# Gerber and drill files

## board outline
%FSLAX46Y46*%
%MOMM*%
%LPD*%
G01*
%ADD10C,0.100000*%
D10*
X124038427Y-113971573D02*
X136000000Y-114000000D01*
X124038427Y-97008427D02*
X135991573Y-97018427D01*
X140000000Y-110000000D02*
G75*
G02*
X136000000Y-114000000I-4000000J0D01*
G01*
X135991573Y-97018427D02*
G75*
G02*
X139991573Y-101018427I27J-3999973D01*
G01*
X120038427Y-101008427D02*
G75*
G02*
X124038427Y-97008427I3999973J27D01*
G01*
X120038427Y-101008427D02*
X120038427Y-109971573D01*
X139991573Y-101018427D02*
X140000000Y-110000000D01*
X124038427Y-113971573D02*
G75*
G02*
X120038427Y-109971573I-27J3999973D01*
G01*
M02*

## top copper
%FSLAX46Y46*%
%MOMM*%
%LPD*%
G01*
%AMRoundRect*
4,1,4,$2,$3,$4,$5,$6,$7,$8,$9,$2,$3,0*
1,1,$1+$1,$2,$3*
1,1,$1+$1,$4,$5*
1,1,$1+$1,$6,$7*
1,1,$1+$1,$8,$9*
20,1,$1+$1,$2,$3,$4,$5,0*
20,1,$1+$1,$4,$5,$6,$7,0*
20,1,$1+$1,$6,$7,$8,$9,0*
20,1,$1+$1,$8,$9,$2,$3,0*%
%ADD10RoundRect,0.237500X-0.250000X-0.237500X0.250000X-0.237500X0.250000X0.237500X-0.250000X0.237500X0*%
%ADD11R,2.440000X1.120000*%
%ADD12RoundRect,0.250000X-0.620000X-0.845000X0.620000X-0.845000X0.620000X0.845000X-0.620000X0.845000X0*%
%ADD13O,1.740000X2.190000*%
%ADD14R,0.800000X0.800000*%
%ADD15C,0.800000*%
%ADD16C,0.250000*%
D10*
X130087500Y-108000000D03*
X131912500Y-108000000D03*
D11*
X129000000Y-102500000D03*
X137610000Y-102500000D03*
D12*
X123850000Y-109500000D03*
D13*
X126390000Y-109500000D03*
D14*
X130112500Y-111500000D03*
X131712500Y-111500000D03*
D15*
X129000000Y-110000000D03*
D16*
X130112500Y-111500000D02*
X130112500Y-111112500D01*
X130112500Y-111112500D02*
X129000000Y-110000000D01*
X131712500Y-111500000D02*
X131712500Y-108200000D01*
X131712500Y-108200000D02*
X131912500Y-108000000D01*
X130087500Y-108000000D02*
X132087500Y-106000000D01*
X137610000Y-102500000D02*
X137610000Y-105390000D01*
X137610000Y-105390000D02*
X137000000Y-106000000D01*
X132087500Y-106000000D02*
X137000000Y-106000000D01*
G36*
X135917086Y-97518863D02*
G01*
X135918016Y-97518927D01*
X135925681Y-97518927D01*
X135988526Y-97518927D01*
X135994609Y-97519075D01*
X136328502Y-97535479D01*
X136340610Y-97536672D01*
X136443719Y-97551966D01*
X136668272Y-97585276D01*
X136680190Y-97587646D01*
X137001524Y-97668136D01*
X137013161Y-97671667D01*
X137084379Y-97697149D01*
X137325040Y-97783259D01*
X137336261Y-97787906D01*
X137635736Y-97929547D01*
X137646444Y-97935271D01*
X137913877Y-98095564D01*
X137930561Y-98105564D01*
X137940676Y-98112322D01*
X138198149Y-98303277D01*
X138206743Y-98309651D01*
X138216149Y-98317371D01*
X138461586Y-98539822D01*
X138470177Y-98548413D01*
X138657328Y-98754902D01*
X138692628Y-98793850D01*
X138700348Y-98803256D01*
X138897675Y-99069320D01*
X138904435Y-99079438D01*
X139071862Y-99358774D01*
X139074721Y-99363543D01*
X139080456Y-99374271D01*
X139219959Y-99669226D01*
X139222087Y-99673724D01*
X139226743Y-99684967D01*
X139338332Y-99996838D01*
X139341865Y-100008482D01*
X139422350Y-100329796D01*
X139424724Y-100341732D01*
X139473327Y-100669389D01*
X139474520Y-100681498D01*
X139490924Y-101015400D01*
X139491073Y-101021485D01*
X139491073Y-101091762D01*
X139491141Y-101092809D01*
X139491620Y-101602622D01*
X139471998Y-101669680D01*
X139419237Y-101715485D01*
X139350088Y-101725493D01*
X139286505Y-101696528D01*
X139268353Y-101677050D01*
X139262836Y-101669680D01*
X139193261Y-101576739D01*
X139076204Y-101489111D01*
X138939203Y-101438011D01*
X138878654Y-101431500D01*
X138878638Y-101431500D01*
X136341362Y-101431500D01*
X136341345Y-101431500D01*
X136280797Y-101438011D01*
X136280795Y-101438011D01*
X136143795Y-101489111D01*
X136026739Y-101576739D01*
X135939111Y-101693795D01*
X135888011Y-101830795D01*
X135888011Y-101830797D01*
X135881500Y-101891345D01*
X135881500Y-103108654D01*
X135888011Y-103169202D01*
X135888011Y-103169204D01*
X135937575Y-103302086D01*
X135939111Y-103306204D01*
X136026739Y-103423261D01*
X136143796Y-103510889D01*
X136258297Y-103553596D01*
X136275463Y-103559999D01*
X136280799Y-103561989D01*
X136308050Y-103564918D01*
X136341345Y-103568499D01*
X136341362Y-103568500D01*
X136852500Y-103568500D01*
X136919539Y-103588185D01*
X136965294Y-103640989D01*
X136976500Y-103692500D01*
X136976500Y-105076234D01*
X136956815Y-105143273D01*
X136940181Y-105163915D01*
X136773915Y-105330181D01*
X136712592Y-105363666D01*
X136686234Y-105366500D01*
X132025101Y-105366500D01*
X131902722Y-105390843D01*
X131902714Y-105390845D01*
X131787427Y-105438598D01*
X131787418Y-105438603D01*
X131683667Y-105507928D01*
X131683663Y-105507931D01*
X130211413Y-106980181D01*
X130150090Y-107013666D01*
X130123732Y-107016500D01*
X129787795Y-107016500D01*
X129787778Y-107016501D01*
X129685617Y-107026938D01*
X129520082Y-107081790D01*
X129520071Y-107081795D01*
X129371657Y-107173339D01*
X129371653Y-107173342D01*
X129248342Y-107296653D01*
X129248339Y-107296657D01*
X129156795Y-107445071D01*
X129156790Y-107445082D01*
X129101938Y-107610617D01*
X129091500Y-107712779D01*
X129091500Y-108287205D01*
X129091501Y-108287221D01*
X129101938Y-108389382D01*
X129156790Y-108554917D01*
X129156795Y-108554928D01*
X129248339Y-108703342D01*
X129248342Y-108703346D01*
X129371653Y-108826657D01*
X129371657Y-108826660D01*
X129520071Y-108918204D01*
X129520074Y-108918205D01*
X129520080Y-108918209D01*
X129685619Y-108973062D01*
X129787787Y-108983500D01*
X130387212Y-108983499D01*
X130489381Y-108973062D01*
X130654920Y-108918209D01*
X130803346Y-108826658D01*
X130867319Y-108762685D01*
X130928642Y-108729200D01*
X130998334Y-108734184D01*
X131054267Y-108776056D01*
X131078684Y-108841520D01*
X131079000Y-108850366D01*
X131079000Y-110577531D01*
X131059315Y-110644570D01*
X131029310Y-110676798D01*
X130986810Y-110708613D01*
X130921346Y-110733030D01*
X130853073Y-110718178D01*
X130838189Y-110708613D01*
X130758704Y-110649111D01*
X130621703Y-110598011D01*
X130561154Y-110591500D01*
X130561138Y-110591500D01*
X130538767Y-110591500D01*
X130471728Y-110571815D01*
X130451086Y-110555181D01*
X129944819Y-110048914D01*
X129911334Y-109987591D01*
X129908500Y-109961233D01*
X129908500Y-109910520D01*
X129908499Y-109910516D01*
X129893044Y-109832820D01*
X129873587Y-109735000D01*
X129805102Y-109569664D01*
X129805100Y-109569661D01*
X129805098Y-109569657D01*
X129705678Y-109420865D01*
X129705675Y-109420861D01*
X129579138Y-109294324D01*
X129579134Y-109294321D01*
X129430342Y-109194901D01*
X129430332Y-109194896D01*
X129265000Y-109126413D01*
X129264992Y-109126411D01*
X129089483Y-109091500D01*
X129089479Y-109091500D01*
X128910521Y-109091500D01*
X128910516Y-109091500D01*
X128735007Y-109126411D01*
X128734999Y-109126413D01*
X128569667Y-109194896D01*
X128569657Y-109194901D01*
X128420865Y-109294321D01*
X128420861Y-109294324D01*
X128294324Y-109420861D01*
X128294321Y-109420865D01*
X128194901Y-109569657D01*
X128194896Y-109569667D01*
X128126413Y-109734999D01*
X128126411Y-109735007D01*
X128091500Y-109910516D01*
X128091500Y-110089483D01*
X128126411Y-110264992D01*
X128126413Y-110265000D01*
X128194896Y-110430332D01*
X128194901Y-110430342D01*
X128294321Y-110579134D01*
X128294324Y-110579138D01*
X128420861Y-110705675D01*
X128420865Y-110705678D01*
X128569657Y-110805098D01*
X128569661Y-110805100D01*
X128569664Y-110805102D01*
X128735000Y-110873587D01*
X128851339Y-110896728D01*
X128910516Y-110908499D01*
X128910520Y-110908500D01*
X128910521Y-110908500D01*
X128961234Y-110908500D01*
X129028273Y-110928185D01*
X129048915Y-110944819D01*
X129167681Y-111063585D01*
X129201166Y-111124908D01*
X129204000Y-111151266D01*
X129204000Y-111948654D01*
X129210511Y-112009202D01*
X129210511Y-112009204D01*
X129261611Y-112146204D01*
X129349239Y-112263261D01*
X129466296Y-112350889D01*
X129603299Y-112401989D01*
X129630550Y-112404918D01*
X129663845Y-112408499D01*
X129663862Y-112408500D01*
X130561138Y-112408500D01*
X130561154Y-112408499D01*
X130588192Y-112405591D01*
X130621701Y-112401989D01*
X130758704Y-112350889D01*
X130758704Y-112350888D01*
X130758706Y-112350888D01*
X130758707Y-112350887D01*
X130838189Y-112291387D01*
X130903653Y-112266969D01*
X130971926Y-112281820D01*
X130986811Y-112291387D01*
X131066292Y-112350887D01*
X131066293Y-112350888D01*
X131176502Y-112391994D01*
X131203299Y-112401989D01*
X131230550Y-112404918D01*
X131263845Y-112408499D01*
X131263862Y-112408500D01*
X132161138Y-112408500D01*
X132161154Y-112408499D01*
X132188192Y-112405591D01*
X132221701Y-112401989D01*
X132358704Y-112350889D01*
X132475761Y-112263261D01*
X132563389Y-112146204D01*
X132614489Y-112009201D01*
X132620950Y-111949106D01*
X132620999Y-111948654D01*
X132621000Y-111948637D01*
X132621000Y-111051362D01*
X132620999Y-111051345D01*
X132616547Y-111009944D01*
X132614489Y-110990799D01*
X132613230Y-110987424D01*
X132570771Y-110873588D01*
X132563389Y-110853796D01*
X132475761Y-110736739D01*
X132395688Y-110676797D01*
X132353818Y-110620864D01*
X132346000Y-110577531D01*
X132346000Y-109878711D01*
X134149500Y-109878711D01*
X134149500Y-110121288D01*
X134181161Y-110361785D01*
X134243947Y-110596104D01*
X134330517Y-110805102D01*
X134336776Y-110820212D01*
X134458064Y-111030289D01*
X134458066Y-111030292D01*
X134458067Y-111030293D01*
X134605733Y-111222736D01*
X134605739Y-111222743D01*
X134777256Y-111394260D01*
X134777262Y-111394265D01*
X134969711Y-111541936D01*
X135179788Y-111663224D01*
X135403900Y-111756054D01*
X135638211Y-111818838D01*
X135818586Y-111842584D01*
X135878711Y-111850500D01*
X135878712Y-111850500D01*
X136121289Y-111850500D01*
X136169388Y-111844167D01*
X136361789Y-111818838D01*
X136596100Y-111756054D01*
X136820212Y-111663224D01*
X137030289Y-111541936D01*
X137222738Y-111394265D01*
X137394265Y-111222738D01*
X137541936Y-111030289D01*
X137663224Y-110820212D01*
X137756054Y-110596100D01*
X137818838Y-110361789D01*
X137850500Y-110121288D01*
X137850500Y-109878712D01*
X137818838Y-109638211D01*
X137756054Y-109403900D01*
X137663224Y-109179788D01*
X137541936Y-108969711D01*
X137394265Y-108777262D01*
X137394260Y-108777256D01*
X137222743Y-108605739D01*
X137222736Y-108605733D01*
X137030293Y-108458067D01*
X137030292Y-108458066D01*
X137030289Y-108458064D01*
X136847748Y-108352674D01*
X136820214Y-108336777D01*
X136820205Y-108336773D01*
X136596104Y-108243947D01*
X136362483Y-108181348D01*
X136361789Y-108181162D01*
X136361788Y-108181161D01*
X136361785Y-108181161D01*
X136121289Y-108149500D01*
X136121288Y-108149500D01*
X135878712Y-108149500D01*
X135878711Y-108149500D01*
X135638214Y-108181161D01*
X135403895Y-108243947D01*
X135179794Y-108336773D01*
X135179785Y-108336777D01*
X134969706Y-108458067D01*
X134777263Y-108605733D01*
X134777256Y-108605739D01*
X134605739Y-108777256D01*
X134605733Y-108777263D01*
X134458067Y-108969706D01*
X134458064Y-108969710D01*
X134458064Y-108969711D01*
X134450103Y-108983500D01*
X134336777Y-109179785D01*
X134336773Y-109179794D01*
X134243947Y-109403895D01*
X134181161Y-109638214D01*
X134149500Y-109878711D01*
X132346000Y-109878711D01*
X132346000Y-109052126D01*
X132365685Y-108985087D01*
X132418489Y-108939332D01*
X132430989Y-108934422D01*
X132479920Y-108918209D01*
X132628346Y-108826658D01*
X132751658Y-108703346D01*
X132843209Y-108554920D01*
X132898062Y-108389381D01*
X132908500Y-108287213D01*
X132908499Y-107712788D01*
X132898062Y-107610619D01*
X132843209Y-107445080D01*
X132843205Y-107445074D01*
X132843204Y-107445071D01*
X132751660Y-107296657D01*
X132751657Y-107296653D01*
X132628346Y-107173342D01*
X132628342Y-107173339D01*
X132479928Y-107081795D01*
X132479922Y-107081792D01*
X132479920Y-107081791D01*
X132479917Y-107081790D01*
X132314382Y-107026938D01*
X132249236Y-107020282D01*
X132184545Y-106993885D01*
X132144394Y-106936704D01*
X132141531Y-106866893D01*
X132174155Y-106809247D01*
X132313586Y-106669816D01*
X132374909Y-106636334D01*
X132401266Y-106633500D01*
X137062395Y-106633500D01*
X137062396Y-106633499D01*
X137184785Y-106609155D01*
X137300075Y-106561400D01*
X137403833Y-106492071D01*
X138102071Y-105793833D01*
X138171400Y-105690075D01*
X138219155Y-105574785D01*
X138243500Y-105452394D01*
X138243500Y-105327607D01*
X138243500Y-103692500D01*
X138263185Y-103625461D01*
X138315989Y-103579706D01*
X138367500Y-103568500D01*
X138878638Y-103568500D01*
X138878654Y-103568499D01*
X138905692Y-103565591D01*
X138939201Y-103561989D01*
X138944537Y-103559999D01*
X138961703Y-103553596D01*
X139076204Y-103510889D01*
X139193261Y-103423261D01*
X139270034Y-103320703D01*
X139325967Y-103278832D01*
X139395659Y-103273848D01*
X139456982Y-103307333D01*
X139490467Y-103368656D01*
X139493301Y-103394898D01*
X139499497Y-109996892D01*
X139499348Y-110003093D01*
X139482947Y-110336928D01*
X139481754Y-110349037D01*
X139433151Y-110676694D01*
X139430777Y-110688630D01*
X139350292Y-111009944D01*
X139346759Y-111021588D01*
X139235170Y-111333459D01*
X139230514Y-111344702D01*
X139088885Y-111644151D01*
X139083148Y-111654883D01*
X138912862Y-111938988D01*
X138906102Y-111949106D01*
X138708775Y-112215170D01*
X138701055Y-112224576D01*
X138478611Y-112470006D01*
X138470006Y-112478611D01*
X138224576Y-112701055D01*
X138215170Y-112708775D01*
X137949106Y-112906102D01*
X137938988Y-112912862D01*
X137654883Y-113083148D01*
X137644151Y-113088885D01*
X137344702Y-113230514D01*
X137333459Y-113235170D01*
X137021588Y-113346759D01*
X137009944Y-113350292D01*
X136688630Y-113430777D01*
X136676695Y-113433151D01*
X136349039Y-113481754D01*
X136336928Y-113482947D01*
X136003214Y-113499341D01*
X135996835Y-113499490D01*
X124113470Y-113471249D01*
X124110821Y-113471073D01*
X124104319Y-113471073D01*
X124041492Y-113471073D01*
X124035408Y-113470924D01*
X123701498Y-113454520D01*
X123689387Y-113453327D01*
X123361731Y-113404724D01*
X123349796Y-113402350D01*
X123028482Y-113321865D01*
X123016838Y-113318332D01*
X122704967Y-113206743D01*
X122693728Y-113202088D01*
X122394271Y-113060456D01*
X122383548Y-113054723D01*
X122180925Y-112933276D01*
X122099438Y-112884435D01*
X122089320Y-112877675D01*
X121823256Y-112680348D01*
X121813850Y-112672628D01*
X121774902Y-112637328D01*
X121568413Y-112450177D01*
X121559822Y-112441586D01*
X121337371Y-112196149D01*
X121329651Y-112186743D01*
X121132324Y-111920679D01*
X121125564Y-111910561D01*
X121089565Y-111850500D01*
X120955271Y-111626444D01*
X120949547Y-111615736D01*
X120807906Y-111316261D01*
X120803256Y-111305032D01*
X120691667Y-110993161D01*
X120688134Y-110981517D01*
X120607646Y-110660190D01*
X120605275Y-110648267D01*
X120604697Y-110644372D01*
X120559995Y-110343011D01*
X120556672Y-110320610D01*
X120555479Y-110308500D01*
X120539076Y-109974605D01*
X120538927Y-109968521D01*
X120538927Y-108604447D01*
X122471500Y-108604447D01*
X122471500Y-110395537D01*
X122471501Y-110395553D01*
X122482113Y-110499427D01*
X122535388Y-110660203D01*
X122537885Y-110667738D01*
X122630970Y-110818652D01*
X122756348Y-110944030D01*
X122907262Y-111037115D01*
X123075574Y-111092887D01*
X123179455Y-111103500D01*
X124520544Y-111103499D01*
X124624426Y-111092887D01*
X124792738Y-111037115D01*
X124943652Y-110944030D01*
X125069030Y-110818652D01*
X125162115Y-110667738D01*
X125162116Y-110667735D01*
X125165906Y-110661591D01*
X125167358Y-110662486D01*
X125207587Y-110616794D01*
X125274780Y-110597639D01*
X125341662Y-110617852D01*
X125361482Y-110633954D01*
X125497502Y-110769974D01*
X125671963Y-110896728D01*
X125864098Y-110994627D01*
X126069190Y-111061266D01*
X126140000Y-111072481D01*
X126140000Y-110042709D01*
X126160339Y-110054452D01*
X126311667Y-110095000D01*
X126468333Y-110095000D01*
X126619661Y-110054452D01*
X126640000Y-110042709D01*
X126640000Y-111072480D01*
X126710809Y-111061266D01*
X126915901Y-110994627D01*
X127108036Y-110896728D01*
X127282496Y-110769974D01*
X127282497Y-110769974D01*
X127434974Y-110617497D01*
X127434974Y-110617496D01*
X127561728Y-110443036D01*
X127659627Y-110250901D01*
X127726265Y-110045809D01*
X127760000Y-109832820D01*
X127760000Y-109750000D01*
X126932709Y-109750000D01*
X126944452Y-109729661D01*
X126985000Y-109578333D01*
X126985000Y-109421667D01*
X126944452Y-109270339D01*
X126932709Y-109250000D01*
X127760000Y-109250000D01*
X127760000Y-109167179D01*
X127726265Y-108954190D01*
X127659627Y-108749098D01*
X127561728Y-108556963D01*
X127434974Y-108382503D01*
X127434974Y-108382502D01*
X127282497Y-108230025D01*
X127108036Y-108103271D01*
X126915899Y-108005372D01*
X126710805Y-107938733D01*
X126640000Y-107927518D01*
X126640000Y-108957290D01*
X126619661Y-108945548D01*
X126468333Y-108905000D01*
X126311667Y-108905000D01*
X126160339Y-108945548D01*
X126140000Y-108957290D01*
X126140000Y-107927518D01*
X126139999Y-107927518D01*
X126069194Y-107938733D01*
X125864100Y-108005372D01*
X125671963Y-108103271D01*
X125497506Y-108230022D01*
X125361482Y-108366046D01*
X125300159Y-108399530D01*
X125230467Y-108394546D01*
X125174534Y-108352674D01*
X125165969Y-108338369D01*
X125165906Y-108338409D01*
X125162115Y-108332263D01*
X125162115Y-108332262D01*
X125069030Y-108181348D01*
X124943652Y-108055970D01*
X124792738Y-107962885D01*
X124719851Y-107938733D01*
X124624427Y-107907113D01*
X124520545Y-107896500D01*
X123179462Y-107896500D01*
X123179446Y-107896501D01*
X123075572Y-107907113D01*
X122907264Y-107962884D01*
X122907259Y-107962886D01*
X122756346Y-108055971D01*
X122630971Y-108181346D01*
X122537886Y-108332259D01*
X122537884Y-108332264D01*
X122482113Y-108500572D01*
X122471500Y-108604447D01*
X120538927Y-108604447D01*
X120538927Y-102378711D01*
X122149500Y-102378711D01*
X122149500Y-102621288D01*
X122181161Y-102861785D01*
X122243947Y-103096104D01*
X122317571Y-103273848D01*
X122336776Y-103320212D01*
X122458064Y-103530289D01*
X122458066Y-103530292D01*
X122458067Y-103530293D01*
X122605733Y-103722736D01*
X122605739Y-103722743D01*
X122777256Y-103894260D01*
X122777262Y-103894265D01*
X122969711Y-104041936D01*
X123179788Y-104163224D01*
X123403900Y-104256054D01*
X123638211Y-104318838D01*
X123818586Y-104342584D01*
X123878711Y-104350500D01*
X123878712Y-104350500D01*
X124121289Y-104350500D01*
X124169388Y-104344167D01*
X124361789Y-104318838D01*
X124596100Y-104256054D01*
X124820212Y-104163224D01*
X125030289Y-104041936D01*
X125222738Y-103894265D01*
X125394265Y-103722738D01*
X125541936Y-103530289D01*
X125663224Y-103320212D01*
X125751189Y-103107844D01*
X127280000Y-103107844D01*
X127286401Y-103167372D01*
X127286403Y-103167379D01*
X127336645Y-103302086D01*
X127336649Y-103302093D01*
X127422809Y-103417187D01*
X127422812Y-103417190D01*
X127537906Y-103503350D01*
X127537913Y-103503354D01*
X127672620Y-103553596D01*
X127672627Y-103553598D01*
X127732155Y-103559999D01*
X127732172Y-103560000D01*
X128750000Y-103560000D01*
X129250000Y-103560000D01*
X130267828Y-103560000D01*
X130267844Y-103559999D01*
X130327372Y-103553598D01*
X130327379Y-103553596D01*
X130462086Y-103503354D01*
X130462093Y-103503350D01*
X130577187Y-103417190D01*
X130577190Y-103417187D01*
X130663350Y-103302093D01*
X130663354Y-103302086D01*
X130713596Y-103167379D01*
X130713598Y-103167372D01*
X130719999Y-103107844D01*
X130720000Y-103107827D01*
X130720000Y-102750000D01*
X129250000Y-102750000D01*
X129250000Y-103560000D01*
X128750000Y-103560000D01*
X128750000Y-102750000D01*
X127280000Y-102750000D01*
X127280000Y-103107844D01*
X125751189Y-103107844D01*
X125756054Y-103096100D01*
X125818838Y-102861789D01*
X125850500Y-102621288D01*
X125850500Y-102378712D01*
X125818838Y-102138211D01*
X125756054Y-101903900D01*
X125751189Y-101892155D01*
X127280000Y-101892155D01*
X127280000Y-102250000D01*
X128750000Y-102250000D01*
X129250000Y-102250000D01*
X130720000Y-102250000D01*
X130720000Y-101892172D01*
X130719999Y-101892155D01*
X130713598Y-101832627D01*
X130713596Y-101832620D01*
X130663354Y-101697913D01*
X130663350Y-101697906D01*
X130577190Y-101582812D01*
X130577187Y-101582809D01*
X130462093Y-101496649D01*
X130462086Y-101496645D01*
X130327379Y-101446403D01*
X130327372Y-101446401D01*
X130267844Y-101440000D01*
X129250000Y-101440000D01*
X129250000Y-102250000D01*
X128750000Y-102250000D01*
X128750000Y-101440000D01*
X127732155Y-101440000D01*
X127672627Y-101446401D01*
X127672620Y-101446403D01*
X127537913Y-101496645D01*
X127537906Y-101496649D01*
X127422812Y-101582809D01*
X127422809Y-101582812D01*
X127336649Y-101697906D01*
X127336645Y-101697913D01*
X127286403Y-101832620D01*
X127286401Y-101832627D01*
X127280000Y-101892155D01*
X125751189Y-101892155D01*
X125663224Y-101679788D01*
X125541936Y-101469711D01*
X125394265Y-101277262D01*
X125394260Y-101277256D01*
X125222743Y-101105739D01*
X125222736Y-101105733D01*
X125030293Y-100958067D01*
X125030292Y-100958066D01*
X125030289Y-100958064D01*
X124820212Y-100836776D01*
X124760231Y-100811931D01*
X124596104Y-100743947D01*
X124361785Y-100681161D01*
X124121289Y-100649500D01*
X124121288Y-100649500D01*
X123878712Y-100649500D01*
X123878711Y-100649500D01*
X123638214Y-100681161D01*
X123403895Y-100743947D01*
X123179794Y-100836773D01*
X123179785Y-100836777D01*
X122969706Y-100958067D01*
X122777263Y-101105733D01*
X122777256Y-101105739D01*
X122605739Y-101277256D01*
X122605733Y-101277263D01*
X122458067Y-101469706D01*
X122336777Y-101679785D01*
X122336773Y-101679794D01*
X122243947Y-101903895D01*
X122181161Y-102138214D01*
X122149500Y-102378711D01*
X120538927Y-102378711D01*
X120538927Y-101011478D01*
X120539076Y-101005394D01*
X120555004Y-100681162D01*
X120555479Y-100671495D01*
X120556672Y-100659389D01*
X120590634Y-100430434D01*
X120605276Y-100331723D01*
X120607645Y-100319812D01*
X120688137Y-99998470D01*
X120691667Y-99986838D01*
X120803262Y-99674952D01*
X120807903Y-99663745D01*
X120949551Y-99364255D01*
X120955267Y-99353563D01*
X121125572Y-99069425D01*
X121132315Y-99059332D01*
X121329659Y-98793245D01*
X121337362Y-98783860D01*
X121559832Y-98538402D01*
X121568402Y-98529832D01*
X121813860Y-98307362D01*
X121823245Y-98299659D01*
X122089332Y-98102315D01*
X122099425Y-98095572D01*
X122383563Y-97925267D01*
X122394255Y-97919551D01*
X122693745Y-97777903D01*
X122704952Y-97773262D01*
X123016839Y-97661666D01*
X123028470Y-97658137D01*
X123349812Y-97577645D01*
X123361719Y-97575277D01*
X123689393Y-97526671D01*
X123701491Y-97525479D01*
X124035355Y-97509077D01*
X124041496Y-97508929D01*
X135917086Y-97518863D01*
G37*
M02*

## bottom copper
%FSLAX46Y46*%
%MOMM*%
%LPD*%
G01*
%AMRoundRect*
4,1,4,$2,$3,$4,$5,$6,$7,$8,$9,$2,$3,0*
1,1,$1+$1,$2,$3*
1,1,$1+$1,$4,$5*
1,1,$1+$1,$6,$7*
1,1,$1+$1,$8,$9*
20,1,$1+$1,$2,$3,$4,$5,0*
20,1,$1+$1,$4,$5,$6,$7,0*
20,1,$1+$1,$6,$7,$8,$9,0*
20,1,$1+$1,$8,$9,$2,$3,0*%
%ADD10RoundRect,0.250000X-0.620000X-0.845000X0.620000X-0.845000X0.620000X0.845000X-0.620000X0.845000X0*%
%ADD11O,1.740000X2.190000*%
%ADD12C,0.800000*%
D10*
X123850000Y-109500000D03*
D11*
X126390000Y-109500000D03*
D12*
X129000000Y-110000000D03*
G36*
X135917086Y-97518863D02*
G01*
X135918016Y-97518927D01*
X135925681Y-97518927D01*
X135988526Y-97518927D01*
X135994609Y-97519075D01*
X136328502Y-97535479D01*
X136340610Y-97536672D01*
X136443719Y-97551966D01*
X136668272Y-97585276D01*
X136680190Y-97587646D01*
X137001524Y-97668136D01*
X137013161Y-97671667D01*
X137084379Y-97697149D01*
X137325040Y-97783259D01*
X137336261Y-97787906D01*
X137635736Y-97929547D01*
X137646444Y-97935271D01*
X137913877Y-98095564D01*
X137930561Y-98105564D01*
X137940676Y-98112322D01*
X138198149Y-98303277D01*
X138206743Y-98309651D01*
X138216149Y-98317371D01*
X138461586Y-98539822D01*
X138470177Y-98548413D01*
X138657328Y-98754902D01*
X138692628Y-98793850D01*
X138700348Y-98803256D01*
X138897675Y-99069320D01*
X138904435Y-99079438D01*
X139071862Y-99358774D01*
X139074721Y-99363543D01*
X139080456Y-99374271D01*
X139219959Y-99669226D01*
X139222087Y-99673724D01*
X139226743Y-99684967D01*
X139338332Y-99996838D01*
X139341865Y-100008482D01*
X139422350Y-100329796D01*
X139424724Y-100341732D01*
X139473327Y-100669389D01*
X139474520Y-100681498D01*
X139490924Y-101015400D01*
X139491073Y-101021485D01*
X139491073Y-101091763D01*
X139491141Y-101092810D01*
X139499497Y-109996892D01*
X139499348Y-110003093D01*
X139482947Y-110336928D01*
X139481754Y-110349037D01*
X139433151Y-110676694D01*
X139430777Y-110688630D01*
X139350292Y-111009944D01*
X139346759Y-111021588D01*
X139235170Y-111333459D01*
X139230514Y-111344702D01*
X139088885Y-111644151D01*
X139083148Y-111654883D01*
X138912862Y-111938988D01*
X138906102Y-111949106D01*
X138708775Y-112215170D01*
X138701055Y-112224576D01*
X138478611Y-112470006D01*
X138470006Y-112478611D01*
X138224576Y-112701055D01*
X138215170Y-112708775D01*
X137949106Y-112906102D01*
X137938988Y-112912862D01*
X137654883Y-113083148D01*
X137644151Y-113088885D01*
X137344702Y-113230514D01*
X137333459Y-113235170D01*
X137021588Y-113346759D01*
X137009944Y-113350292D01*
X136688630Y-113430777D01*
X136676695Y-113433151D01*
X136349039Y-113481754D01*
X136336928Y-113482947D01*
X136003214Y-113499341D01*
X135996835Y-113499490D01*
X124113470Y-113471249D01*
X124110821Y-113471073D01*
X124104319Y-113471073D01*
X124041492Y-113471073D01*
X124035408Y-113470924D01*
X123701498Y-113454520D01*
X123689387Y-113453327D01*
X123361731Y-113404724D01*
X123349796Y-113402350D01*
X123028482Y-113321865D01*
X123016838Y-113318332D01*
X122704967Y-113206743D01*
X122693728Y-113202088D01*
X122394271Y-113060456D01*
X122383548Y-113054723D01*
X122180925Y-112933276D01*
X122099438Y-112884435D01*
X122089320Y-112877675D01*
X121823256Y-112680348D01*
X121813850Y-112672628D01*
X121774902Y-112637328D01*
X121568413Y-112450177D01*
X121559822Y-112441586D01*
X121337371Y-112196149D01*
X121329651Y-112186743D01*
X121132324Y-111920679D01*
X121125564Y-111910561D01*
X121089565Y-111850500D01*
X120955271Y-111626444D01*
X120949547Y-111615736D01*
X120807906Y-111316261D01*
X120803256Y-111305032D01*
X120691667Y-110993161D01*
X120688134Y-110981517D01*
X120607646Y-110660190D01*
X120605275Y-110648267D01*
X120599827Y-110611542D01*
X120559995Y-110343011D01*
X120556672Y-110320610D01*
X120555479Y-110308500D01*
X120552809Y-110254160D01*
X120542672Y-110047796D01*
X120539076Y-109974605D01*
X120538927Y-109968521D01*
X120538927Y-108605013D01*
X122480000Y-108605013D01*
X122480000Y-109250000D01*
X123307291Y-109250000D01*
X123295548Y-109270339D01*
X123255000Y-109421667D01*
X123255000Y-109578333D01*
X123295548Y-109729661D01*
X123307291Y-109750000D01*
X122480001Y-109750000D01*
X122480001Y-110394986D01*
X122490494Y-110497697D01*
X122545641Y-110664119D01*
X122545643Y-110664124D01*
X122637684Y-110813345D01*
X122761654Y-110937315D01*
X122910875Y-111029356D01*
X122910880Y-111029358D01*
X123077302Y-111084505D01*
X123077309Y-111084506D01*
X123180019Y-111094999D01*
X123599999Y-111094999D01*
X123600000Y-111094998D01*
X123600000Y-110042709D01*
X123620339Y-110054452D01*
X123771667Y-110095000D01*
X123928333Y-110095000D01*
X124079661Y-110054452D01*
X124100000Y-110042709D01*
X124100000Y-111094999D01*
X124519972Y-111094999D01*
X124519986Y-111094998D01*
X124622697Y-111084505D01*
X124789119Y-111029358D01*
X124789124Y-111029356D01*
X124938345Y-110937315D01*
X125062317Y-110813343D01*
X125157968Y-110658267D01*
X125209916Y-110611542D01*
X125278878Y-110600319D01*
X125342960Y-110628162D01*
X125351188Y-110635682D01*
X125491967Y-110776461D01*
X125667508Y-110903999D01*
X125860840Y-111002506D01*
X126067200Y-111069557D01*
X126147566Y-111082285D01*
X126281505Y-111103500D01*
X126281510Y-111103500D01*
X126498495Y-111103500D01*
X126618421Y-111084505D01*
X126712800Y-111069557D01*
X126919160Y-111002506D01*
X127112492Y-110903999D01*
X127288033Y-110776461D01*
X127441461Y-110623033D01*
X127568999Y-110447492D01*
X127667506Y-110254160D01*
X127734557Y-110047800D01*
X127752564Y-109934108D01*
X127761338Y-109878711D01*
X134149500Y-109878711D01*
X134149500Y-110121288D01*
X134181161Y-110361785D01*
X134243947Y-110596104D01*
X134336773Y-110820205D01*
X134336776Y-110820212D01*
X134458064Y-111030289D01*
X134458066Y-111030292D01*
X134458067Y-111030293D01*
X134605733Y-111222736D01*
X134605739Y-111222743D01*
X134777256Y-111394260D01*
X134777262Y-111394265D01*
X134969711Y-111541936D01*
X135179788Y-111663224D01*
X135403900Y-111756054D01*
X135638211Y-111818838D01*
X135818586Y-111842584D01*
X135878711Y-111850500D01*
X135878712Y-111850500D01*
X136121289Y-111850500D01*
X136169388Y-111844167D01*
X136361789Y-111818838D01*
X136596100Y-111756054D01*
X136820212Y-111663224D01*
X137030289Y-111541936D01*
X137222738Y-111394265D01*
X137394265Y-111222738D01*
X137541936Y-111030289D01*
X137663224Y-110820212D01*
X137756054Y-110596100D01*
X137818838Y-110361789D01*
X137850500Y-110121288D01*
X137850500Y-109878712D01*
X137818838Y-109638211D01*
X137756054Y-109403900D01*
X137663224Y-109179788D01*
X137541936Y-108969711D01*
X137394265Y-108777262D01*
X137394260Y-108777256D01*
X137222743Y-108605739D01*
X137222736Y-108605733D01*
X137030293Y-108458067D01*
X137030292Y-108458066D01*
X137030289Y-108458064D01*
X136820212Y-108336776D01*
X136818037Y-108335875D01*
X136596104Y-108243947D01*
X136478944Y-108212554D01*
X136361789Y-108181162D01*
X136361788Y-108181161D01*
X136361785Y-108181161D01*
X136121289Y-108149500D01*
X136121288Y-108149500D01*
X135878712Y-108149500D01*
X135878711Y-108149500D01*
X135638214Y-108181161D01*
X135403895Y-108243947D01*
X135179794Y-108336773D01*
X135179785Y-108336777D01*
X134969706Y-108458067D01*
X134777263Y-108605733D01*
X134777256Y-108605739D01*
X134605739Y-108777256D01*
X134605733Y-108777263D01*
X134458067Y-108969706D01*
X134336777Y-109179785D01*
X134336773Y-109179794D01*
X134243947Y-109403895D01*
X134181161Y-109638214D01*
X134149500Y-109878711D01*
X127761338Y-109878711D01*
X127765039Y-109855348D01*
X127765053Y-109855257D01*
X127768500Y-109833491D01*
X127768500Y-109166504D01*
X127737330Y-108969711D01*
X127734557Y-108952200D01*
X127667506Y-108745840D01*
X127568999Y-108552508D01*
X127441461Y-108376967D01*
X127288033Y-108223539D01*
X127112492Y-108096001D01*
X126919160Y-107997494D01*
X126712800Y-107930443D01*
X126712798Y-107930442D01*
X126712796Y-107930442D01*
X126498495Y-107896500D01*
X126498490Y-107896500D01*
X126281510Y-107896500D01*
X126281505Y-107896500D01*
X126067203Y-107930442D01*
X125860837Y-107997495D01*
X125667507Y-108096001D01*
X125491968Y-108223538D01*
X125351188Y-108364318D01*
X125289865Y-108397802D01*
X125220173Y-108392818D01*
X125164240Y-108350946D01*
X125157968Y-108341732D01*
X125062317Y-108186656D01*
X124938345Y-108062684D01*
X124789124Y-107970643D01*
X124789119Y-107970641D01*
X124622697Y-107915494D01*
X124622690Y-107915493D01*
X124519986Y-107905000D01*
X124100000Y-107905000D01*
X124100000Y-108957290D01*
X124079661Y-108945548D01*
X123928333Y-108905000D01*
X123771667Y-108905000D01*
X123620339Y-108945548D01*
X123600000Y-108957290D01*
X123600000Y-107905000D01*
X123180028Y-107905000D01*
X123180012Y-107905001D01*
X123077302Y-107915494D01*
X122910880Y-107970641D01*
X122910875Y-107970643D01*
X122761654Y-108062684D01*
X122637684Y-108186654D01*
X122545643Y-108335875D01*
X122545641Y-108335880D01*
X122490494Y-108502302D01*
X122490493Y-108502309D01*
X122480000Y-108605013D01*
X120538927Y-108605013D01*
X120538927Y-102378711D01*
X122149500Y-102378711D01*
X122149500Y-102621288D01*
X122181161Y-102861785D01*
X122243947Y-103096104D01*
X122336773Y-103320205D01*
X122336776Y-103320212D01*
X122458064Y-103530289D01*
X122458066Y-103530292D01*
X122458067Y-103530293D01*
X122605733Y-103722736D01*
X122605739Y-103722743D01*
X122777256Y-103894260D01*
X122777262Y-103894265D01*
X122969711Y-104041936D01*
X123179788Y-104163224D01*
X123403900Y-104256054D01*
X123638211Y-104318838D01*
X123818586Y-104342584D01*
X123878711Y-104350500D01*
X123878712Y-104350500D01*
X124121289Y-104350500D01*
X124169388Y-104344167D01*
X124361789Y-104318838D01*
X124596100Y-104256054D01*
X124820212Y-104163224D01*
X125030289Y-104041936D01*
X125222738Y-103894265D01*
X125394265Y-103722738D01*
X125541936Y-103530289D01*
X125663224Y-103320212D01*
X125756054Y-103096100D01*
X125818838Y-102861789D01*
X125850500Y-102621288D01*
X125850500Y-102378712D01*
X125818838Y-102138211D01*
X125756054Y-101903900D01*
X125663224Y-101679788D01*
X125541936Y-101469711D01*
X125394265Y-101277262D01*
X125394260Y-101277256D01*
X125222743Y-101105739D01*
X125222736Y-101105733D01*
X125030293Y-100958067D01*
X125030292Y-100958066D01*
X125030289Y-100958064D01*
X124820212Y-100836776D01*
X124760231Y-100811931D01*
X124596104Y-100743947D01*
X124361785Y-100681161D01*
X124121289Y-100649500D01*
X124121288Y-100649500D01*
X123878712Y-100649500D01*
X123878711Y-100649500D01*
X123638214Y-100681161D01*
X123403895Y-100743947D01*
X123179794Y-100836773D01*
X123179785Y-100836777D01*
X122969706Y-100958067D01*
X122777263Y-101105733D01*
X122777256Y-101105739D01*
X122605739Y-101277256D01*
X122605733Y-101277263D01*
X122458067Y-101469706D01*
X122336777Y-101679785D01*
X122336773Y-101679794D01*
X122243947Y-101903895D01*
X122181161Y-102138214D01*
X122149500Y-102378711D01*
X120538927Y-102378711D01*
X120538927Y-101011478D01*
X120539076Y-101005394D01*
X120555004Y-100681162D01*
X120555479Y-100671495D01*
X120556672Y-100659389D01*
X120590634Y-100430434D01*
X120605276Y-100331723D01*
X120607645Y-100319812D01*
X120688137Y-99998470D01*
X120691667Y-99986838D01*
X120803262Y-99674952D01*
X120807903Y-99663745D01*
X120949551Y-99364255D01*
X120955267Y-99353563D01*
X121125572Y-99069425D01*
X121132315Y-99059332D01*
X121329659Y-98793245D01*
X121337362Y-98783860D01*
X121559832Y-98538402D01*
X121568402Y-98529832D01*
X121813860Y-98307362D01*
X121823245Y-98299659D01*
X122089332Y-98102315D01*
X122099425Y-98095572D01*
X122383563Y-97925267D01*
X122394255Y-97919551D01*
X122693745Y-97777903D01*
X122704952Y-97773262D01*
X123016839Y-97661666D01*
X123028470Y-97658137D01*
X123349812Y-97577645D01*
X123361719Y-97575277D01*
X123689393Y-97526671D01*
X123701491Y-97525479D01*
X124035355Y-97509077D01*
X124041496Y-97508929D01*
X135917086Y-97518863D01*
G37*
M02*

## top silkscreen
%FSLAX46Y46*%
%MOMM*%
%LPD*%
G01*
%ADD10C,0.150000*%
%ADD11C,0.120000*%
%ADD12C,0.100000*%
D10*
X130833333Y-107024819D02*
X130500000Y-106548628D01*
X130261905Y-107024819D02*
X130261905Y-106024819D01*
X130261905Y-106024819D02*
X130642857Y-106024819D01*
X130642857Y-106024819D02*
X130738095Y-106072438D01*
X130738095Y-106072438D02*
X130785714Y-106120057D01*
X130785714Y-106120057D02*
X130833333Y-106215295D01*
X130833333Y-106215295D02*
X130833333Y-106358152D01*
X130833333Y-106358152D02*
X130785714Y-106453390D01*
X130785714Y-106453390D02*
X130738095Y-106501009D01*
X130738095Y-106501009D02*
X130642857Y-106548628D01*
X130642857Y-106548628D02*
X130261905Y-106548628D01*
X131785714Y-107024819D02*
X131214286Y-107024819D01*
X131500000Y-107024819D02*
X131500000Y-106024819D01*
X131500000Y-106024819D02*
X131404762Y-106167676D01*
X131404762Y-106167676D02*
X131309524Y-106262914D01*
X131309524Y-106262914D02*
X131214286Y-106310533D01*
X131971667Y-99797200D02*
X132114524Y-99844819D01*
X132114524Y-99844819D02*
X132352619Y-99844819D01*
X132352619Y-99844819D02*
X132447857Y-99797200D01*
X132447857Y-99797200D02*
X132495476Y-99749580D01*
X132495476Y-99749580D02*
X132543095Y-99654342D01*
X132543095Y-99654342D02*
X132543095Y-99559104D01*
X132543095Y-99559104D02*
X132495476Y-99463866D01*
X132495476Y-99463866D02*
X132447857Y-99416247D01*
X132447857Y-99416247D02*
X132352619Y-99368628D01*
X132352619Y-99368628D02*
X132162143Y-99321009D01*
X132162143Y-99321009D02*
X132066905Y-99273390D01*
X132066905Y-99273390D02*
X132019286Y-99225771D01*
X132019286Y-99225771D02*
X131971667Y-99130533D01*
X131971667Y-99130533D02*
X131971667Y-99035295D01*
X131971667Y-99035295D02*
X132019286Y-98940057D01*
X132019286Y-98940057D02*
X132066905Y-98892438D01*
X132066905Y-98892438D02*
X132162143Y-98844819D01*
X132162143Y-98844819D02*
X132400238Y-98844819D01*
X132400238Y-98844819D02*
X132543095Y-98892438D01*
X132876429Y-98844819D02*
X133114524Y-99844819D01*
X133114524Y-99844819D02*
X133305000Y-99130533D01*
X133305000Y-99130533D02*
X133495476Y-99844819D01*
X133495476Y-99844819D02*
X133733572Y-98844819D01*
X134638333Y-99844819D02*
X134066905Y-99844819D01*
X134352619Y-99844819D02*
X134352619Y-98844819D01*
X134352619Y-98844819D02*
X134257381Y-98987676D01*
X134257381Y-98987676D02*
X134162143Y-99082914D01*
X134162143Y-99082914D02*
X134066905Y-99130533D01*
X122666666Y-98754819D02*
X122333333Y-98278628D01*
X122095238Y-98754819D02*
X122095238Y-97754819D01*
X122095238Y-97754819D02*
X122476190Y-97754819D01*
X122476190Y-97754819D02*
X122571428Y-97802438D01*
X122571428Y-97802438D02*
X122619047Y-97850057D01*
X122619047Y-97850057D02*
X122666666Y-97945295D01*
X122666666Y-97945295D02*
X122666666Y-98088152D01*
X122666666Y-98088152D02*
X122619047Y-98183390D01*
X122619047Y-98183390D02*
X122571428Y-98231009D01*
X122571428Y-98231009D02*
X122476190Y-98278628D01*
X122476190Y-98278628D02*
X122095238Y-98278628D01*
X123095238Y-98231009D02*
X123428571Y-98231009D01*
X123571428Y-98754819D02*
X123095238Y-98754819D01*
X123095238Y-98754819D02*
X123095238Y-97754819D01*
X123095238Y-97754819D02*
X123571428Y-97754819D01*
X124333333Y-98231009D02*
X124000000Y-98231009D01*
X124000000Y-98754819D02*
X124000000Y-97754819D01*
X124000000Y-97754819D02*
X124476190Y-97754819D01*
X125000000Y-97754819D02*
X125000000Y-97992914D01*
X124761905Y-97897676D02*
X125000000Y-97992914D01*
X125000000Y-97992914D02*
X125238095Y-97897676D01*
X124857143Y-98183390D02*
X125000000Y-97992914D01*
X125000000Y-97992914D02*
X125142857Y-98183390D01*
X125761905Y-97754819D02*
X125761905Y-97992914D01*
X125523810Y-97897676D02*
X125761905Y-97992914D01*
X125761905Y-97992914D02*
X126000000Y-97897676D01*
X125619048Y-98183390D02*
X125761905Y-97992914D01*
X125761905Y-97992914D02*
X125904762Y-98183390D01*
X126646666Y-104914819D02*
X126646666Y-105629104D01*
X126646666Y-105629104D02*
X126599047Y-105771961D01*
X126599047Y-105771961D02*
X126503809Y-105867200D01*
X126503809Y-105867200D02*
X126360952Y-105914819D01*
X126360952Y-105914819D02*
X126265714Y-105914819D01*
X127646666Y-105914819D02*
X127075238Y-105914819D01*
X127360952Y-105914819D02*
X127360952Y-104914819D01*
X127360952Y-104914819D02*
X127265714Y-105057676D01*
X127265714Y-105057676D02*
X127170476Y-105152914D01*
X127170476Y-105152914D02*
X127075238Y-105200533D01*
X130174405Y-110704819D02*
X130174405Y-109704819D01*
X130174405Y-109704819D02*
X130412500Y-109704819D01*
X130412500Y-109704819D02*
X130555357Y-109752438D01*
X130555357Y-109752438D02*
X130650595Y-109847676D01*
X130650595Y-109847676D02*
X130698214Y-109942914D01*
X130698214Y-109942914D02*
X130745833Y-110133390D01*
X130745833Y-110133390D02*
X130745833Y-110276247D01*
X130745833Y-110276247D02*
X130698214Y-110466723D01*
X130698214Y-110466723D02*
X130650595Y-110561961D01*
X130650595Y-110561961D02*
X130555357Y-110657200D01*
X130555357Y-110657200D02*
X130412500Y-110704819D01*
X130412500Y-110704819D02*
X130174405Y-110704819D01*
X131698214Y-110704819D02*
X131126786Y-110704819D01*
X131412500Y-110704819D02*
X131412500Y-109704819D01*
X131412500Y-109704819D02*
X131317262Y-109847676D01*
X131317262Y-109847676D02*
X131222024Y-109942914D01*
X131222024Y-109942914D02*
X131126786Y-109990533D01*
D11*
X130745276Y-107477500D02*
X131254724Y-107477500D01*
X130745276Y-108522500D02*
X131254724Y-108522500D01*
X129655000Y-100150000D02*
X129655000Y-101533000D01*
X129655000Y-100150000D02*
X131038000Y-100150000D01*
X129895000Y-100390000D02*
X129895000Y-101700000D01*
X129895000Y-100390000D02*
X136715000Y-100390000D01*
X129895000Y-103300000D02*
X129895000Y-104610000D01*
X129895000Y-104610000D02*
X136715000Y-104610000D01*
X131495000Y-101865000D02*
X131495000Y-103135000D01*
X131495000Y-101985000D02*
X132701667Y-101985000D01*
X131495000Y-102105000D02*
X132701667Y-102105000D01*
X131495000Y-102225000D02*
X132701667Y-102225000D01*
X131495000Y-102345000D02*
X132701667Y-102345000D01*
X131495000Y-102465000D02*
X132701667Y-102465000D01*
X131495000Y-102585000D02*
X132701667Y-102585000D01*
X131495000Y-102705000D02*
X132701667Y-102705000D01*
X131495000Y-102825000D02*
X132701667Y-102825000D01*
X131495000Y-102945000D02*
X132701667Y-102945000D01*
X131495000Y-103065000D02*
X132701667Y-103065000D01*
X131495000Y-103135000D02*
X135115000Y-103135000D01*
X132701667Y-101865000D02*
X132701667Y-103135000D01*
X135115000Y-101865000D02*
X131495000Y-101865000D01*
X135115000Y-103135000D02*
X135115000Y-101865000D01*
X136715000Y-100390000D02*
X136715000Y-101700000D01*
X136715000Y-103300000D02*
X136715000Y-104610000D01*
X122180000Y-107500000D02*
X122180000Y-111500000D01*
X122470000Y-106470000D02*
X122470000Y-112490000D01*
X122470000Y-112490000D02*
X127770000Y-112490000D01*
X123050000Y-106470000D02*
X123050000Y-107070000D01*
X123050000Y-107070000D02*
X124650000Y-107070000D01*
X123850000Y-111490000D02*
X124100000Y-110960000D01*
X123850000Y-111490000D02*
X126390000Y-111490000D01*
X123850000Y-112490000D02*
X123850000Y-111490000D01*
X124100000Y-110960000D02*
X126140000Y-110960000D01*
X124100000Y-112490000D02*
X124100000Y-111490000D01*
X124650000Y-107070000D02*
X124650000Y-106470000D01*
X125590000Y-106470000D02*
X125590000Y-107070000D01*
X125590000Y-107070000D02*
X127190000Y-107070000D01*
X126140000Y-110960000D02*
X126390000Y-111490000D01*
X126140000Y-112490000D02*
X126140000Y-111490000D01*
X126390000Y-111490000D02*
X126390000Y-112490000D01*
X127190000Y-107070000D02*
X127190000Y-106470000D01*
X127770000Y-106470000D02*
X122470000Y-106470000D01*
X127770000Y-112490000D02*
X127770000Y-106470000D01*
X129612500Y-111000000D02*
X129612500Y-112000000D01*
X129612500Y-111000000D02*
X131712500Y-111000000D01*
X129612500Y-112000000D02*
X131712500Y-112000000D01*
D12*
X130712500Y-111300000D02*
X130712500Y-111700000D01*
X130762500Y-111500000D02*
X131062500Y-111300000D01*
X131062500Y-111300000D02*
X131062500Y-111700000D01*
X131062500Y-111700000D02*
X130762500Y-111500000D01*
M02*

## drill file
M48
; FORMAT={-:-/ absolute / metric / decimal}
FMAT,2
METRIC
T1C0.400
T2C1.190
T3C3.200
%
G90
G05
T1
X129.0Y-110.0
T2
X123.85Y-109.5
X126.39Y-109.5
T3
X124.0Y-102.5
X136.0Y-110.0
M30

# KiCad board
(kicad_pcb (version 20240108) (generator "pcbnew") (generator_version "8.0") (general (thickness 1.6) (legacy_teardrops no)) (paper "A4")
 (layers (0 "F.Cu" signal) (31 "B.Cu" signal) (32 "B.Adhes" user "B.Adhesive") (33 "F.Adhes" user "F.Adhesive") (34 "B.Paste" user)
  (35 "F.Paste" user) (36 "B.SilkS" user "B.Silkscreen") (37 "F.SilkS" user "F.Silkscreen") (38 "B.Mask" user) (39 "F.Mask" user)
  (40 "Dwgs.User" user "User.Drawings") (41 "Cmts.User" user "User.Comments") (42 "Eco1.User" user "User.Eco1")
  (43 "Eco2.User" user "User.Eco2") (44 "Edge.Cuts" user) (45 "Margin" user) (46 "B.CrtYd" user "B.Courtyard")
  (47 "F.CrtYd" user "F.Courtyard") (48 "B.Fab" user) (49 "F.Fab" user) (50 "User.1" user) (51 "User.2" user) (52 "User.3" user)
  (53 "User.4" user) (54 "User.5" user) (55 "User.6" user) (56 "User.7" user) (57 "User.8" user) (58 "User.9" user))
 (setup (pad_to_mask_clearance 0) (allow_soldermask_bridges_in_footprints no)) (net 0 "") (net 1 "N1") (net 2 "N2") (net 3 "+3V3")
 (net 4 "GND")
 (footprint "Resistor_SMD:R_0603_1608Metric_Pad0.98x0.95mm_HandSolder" (layer "F.Cu") (at 131 108)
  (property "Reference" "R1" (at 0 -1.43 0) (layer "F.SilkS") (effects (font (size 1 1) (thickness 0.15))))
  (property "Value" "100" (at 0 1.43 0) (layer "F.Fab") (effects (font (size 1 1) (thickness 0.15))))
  (fp_line (start -0.254724 -0.5225) (end 0.254724 -0.5225) (stroke (width 0.12) (type solid)) (layer "F.SilkS"))
  (fp_line (start -0.254724 0.5225) (end 0.254724 0.5225) (stroke (width 0.12) (type solid)) (layer "F.SilkS"))
  (pad "1" smd roundrect (at -0.9125 0) (size 0.975 0.95) (layers "F.Cu" "F.Paste" "F.Mask") (roundrect_rratio 0.25) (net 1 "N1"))
  (pad "2" smd roundrect (at 0.9125 0) (size 0.975 0.95) (layers "F.Cu" "F.Paste" "F.Mask") (roundrect_rratio 0.25) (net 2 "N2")))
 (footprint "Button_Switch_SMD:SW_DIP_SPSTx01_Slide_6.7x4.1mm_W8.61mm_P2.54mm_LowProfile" (layer "F.Cu") (at 133.305 102.5)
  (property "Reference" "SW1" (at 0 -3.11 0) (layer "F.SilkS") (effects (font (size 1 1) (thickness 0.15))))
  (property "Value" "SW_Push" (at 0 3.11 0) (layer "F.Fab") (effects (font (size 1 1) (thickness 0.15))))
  (fp_line (start -3.65 -2.35) (end -3.65 -0.967) (stroke (width 0.12) (type solid)) (layer "F.SilkS"))
  (fp_line (start -3.65 -2.35) (end -2.267 -2.35) (stroke (width 0.12) (type solid)) (layer "F.SilkS"))
  (fp_line (start -3.41 -2.11) (end -3.41 -0.8) (stroke (width 0.12) (type solid)) (layer "F.SilkS"))
  (fp_line (start -3.41 -2.11) (end 3.41 -2.11) (stroke (width 0.12) (type solid)) (layer "F.SilkS"))
  (fp_line (start -3.41 0.8) (end -3.41 2.11) (stroke (width 0.12) (type solid)) (layer "F.SilkS"))
  (fp_line (start -3.41 2.11) (end 3.41 2.11) (stroke (width 0.12) (type solid)) (layer "F.SilkS"))
  (fp_line (start -1.81 -0.635) (end -1.81 0.635) (stroke (width 0.12) (type solid)) (layer "F.SilkS"))
  (fp_line (start -1.81 -0.515) (end -0.603333 -0.515) (stroke (width 0.12) (type solid)) (layer "F.SilkS"))
  (fp_line (start -1.81 -0.395) (end -0.603333 -0.395) (stroke (width 0.12) (type solid)) (layer "F.SilkS"))
  (fp_line (start -1.81 -0.275) (end -0.603333 -0.275) (stroke (width 0.12) (type solid)) (layer "F.SilkS"))
  (fp_line (start -1.81 -0.155) (end -0.603333 -0.155) (stroke (width 0.12) (type solid)) (layer "F.SilkS"))
  (fp_line (start -1.81 -0.035) (end -0.603333 -0.035) (stroke (width 0.12) (type solid)) (layer "F.SilkS"))
  (fp_line (start -1.81 0.085) (end -0.603333 0.085) (stroke (width 0.12) (type solid)) (layer "F.SilkS"))
  (fp_line (start -1.81 0.205) (end -0.603333 0.205) (stroke (width 0.12) (type solid)) (layer "F.SilkS"))
  (fp_line (start -1.81 0.325) (end -0.603333 0.325) (stroke (width 0.12) (type solid)) (layer "F.SilkS"))
  (fp_line (start -1.81 0.445) (end -0.603333 0.445) (stroke (width 0.12) (type solid)) (layer "F.SilkS"))
  (fp_line (start -1.81 0.565) (end -0.603333 0.565) (stroke (width 0.12) (type solid)) (layer "F.SilkS"))
  (fp_line (start -1.81 0.635) (end 1.81 0.635) (stroke (width 0.12) (type solid)) (layer "F.SilkS"))
  (fp_line (start -0.603333 -0.635) (end -0.603333 0.635) (stroke (width 0.12) (type solid)) (layer "F.SilkS"))
  (fp_line (start 1.81 -0.635) (end -1.81 -0.635) (stroke (width 0.12) (type solid)) (layer "F.SilkS"))
  (fp_line (start 1.81 0.635) (end 1.81 -0.635) (stroke (width 0.12) (type solid)) (layer "F.SilkS"))
  (fp_line (start 3.41 -2.11) (end 3.41 -0.8) (stroke (width 0.12) (type solid)) (layer "F.SilkS"))
  (fp_line (start 3.41 0.8) (end 3.41 2.11) (stroke (width 0.12) (type solid)) (layer "F.SilkS"))
  (pad "1" smd rect (at -4.305 0) (size 2.44 1.12) (layers "F.Cu" "F.Paste" "F.Mask") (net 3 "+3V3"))
  (pad "2" smd rect (at 4.305 0) (size 2.44 1.12) (layers "F.Cu" "F.Paste" "F.Mask") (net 1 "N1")))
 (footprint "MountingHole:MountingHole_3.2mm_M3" (layer "F.Cu") (at 136 110)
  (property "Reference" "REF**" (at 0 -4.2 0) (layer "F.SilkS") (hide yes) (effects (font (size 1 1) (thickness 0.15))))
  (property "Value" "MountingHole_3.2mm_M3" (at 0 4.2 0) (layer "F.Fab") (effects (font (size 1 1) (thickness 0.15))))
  (pad "" np_thru_hole circle (at 0 0) (size 3.2 3.2) (drill 3.2) (layers "*.Cu" "*.Mask")))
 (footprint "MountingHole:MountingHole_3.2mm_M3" (layer "F.Cu") (at 124 102.5)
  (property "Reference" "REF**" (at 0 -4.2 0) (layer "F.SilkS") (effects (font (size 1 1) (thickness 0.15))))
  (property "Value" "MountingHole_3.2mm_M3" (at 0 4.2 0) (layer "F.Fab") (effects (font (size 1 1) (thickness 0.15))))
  (pad "" np_thru_hole circle (at 0 0) (size 3.2 3.2) (drill 3.2) (layers "*.Cu" "*.Mask")))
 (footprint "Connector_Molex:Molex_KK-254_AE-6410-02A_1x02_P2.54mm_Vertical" (layer "F.Cu") (at 123.85 109.5)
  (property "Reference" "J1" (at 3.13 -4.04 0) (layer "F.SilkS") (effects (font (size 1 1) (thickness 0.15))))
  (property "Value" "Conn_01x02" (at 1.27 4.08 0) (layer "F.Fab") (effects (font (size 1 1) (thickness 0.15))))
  (fp_line (start -1.67 -2) (end -1.67 2) (stroke (width 0.12) (type solid)) (layer "F.SilkS"))
  (fp_line (start -1.38 -3.03) (end -1.38 2.99) (stroke (width 0.12) (type solid)) (layer "F.SilkS"))
  (fp_line (start -1.38 2.99) (end 3.92 2.99) (stroke (width 0.12) (type solid)) (layer "F.SilkS"))
  (fp_line (start -0.8 -3.03) (end -0.8 -2.43) (stroke (width 0.12) (type solid)) (layer "F.SilkS"))
  (fp_line (start -0.8 -2.43) (end 0.8 -2.43) (stroke (width 0.12) (type solid)) (layer "F.SilkS"))
  (fp_line (start 0 1.99) (end 0.25 1.46) (stroke (width 0.12) (type solid)) (layer "F.SilkS"))
  (fp_line (start 0 1.99) (end 2.54 1.99) (stroke (width 0.12) (type solid)) (layer "F.SilkS"))
  (fp_line (start 0 2.99) (end 0 1.99) (stroke (width 0.12) (type solid)) (layer "F.SilkS"))
  (fp_line (start 0.25 1.46) (end 2.29 1.46) (stroke (width 0.12) (type solid)) (layer "F.SilkS"))
  (fp_line (start 0.25 2.99) (end 0.25 1.99) (stroke (width 0.12) (type solid)) (layer "F.SilkS"))
  (fp_line (start 0.8 -2.43) (end 0.8 -3.03) (stroke (width 0.12) (type solid)) (layer "F.SilkS"))
  (fp_line (start 1.74 -3.03) (end 1.74 -2.43) (stroke (width 0.12) (type solid)) (layer "F.SilkS"))
  (fp_line (start 1.74 -2.43) (end 3.34 -2.43) (stroke (width 0.12) (type solid)) (layer "F.SilkS"))
  (fp_line (start 2.29 1.46) (end 2.54 1.99) (stroke (width 0.12) (type solid)) (layer "F.SilkS"))
  (fp_line (start 2.29 2.99) (end 2.29 1.99) (stroke (width 0.12) (type solid)) (layer "F.SilkS"))
  (fp_line (start 2.54 1.99) (end 2.54 2.99) (stroke (width 0.12) (type solid)) (layer "F.SilkS"))
  (fp_line (start 3.34 -2.43) (end 3.34 -3.03) (stroke (width 0.12) (type solid)) (layer "F.SilkS"))
  (fp_line (start 3.92 -3.03) (end -1.38 -3.03) (stroke (width 0.12) (type solid)) (layer "F.SilkS"))
  (fp_line (start 3.92 2.99) (end 3.92 -3.03) (stroke (width 0.12) (type solid)) (layer "F.SilkS"))
  (pad "1" thru_hole roundrect (at 0 0) (size 1.74 2.19) (drill 1.19) (layers "*.Cu" "*.Mask") (remove_unused_layers no)
   (roundrect_rratio 0.143678) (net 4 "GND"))
  (pad "2" thru_hole oval (at 2.54 0) (size 1.74 2.19) (drill 1.19) (layers "*.Cu" "*.Mask") (remove_unused_layers no) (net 3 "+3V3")))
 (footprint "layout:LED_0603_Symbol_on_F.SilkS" (layer "F.Cu") (at 130.9125 111.5)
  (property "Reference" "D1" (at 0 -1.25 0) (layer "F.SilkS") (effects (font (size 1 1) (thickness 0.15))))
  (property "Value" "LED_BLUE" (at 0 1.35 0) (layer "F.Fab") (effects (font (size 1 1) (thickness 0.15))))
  (fp_line (start -1.3 -0.5) (end -1.3 0.5) (stroke (width 0.12) (type solid)) (layer "F.SilkS"))
  (fp_line (start -1.3 -0.5) (end 0.8 -0.5) (stroke (width 0.12) (type solid)) (layer "F.SilkS"))
  (fp_line (start -1.3 0.5) (end 0.8 0.5) (stroke (width 0.12) (type solid)) (layer "F.SilkS"))
  (fp_line (start -0.2 -0.2) (end -0.2 0.2) (stroke (width 0.1) (type solid)) (layer "F.SilkS"))
  (fp_line (start -0.15 0) (end 0.15 -0.2) (stroke (width 0.1) (type solid)) (layer "F.SilkS"))
  (fp_line (start 0.15 -0.2) (end 0.15 0.2) (stroke (width 0.1) (type solid)) (layer "F.SilkS"))
  (fp_line (start 0.15 0.2) (end -0.15 0) (stroke (width 0.1) (type solid)) (layer "F.SilkS"))
  (pad "1" smd rect (at -0.8 0 180) (size 0.8 0.8) (layers "F.Cu" "F.Paste" "F.Mask") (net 4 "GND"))
  (pad "2" smd rect (at 0.8 0 180) (size 0.8 0.8) (layers "F.Cu" "F.Paste" "F.Mask") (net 2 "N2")))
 (gr_line (start 124.038427 113.971573) (end 136 114) (stroke (width 0.1) (type default)) (layer "Edge.Cuts"))
 (gr_line (start 124.038427 97.008427) (end 135.991573 97.018427) (stroke (width 0.1) (type default)) (layer "Edge.Cuts"))
 (gr_arc (start 140 110) (mid 138.828427 112.828427) (end 136 114) (stroke (width 0.1) (type default)) (layer "Edge.Cuts"))
 (gr_arc (start 135.991573 97.018427) (mid 138.82 98.19) (end 139.991573 101.018427) (stroke (width 0.1) (type default)) (layer "Edge.Cuts"))
 (gr_arc (start 120.038427 101.008427) (mid 121.21 98.18) (end 124.038427 97.008427) (stroke (width 0.1) (type default)) (layer "Edge.Cuts"))
 (gr_line (start 120.038427 101.008427) (end 120.038427 109.971573) (stroke (width 0.1) (type default)) (layer "Edge.Cuts"))
 (gr_line (start 139.991573 101.018427) (end 140 110) (stroke (width 0.1) (type default)) (layer "Edge.Cuts"))
 (gr_arc (start 124.038427 113.971573) (mid 121.21 112.8) (end 120.038427 109.971573) (stroke (width 0.1) (type default))
  (layer "Edge.Cuts"))
 (segment (start 130.1125 111.5) (end 130.1125 111.1125) (width 0.25) (layer "F.Cu") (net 4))
 (segment (start 130.1125 111.1125) (end 129 110) (width 0.25) (layer "F.Cu") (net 4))
 (via (at 129 110) (size 0.8) (drill 0.4) (layers "F.Cu" "B.Cu") (free yes) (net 4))
 (segment (start 131.7125 111.5) (end 131.7125 108.2) (width 0.25) (layer "F.Cu") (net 2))
 (segment (start 131.7125 108.2) (end 131.9125 108) (width 0.25) (layer "F.Cu") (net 2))
 (segment (start 130.0875 108) (end 132.0875 106) (width 0.25) (layer "F.Cu") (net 1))
 (segment (start 137.61 102.5) (end 137.61 105.39) (width 0.25) (layer "F.Cu") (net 1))
 (segment (start 137.61 105.39) (end 137 106) (width 0.25) (layer "F.Cu") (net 1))
 (segment (start 132.0875 106) (end 137 106) (width 0.25) (layer "F.Cu") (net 1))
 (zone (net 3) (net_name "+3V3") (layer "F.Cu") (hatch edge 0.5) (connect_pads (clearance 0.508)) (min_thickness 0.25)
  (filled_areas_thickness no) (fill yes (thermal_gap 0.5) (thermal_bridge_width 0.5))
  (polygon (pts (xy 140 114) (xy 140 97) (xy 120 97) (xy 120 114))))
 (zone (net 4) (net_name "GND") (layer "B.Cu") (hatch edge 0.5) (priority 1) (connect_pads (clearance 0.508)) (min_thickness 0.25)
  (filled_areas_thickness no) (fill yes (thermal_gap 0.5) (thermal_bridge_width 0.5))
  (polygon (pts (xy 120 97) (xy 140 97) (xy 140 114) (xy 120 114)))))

